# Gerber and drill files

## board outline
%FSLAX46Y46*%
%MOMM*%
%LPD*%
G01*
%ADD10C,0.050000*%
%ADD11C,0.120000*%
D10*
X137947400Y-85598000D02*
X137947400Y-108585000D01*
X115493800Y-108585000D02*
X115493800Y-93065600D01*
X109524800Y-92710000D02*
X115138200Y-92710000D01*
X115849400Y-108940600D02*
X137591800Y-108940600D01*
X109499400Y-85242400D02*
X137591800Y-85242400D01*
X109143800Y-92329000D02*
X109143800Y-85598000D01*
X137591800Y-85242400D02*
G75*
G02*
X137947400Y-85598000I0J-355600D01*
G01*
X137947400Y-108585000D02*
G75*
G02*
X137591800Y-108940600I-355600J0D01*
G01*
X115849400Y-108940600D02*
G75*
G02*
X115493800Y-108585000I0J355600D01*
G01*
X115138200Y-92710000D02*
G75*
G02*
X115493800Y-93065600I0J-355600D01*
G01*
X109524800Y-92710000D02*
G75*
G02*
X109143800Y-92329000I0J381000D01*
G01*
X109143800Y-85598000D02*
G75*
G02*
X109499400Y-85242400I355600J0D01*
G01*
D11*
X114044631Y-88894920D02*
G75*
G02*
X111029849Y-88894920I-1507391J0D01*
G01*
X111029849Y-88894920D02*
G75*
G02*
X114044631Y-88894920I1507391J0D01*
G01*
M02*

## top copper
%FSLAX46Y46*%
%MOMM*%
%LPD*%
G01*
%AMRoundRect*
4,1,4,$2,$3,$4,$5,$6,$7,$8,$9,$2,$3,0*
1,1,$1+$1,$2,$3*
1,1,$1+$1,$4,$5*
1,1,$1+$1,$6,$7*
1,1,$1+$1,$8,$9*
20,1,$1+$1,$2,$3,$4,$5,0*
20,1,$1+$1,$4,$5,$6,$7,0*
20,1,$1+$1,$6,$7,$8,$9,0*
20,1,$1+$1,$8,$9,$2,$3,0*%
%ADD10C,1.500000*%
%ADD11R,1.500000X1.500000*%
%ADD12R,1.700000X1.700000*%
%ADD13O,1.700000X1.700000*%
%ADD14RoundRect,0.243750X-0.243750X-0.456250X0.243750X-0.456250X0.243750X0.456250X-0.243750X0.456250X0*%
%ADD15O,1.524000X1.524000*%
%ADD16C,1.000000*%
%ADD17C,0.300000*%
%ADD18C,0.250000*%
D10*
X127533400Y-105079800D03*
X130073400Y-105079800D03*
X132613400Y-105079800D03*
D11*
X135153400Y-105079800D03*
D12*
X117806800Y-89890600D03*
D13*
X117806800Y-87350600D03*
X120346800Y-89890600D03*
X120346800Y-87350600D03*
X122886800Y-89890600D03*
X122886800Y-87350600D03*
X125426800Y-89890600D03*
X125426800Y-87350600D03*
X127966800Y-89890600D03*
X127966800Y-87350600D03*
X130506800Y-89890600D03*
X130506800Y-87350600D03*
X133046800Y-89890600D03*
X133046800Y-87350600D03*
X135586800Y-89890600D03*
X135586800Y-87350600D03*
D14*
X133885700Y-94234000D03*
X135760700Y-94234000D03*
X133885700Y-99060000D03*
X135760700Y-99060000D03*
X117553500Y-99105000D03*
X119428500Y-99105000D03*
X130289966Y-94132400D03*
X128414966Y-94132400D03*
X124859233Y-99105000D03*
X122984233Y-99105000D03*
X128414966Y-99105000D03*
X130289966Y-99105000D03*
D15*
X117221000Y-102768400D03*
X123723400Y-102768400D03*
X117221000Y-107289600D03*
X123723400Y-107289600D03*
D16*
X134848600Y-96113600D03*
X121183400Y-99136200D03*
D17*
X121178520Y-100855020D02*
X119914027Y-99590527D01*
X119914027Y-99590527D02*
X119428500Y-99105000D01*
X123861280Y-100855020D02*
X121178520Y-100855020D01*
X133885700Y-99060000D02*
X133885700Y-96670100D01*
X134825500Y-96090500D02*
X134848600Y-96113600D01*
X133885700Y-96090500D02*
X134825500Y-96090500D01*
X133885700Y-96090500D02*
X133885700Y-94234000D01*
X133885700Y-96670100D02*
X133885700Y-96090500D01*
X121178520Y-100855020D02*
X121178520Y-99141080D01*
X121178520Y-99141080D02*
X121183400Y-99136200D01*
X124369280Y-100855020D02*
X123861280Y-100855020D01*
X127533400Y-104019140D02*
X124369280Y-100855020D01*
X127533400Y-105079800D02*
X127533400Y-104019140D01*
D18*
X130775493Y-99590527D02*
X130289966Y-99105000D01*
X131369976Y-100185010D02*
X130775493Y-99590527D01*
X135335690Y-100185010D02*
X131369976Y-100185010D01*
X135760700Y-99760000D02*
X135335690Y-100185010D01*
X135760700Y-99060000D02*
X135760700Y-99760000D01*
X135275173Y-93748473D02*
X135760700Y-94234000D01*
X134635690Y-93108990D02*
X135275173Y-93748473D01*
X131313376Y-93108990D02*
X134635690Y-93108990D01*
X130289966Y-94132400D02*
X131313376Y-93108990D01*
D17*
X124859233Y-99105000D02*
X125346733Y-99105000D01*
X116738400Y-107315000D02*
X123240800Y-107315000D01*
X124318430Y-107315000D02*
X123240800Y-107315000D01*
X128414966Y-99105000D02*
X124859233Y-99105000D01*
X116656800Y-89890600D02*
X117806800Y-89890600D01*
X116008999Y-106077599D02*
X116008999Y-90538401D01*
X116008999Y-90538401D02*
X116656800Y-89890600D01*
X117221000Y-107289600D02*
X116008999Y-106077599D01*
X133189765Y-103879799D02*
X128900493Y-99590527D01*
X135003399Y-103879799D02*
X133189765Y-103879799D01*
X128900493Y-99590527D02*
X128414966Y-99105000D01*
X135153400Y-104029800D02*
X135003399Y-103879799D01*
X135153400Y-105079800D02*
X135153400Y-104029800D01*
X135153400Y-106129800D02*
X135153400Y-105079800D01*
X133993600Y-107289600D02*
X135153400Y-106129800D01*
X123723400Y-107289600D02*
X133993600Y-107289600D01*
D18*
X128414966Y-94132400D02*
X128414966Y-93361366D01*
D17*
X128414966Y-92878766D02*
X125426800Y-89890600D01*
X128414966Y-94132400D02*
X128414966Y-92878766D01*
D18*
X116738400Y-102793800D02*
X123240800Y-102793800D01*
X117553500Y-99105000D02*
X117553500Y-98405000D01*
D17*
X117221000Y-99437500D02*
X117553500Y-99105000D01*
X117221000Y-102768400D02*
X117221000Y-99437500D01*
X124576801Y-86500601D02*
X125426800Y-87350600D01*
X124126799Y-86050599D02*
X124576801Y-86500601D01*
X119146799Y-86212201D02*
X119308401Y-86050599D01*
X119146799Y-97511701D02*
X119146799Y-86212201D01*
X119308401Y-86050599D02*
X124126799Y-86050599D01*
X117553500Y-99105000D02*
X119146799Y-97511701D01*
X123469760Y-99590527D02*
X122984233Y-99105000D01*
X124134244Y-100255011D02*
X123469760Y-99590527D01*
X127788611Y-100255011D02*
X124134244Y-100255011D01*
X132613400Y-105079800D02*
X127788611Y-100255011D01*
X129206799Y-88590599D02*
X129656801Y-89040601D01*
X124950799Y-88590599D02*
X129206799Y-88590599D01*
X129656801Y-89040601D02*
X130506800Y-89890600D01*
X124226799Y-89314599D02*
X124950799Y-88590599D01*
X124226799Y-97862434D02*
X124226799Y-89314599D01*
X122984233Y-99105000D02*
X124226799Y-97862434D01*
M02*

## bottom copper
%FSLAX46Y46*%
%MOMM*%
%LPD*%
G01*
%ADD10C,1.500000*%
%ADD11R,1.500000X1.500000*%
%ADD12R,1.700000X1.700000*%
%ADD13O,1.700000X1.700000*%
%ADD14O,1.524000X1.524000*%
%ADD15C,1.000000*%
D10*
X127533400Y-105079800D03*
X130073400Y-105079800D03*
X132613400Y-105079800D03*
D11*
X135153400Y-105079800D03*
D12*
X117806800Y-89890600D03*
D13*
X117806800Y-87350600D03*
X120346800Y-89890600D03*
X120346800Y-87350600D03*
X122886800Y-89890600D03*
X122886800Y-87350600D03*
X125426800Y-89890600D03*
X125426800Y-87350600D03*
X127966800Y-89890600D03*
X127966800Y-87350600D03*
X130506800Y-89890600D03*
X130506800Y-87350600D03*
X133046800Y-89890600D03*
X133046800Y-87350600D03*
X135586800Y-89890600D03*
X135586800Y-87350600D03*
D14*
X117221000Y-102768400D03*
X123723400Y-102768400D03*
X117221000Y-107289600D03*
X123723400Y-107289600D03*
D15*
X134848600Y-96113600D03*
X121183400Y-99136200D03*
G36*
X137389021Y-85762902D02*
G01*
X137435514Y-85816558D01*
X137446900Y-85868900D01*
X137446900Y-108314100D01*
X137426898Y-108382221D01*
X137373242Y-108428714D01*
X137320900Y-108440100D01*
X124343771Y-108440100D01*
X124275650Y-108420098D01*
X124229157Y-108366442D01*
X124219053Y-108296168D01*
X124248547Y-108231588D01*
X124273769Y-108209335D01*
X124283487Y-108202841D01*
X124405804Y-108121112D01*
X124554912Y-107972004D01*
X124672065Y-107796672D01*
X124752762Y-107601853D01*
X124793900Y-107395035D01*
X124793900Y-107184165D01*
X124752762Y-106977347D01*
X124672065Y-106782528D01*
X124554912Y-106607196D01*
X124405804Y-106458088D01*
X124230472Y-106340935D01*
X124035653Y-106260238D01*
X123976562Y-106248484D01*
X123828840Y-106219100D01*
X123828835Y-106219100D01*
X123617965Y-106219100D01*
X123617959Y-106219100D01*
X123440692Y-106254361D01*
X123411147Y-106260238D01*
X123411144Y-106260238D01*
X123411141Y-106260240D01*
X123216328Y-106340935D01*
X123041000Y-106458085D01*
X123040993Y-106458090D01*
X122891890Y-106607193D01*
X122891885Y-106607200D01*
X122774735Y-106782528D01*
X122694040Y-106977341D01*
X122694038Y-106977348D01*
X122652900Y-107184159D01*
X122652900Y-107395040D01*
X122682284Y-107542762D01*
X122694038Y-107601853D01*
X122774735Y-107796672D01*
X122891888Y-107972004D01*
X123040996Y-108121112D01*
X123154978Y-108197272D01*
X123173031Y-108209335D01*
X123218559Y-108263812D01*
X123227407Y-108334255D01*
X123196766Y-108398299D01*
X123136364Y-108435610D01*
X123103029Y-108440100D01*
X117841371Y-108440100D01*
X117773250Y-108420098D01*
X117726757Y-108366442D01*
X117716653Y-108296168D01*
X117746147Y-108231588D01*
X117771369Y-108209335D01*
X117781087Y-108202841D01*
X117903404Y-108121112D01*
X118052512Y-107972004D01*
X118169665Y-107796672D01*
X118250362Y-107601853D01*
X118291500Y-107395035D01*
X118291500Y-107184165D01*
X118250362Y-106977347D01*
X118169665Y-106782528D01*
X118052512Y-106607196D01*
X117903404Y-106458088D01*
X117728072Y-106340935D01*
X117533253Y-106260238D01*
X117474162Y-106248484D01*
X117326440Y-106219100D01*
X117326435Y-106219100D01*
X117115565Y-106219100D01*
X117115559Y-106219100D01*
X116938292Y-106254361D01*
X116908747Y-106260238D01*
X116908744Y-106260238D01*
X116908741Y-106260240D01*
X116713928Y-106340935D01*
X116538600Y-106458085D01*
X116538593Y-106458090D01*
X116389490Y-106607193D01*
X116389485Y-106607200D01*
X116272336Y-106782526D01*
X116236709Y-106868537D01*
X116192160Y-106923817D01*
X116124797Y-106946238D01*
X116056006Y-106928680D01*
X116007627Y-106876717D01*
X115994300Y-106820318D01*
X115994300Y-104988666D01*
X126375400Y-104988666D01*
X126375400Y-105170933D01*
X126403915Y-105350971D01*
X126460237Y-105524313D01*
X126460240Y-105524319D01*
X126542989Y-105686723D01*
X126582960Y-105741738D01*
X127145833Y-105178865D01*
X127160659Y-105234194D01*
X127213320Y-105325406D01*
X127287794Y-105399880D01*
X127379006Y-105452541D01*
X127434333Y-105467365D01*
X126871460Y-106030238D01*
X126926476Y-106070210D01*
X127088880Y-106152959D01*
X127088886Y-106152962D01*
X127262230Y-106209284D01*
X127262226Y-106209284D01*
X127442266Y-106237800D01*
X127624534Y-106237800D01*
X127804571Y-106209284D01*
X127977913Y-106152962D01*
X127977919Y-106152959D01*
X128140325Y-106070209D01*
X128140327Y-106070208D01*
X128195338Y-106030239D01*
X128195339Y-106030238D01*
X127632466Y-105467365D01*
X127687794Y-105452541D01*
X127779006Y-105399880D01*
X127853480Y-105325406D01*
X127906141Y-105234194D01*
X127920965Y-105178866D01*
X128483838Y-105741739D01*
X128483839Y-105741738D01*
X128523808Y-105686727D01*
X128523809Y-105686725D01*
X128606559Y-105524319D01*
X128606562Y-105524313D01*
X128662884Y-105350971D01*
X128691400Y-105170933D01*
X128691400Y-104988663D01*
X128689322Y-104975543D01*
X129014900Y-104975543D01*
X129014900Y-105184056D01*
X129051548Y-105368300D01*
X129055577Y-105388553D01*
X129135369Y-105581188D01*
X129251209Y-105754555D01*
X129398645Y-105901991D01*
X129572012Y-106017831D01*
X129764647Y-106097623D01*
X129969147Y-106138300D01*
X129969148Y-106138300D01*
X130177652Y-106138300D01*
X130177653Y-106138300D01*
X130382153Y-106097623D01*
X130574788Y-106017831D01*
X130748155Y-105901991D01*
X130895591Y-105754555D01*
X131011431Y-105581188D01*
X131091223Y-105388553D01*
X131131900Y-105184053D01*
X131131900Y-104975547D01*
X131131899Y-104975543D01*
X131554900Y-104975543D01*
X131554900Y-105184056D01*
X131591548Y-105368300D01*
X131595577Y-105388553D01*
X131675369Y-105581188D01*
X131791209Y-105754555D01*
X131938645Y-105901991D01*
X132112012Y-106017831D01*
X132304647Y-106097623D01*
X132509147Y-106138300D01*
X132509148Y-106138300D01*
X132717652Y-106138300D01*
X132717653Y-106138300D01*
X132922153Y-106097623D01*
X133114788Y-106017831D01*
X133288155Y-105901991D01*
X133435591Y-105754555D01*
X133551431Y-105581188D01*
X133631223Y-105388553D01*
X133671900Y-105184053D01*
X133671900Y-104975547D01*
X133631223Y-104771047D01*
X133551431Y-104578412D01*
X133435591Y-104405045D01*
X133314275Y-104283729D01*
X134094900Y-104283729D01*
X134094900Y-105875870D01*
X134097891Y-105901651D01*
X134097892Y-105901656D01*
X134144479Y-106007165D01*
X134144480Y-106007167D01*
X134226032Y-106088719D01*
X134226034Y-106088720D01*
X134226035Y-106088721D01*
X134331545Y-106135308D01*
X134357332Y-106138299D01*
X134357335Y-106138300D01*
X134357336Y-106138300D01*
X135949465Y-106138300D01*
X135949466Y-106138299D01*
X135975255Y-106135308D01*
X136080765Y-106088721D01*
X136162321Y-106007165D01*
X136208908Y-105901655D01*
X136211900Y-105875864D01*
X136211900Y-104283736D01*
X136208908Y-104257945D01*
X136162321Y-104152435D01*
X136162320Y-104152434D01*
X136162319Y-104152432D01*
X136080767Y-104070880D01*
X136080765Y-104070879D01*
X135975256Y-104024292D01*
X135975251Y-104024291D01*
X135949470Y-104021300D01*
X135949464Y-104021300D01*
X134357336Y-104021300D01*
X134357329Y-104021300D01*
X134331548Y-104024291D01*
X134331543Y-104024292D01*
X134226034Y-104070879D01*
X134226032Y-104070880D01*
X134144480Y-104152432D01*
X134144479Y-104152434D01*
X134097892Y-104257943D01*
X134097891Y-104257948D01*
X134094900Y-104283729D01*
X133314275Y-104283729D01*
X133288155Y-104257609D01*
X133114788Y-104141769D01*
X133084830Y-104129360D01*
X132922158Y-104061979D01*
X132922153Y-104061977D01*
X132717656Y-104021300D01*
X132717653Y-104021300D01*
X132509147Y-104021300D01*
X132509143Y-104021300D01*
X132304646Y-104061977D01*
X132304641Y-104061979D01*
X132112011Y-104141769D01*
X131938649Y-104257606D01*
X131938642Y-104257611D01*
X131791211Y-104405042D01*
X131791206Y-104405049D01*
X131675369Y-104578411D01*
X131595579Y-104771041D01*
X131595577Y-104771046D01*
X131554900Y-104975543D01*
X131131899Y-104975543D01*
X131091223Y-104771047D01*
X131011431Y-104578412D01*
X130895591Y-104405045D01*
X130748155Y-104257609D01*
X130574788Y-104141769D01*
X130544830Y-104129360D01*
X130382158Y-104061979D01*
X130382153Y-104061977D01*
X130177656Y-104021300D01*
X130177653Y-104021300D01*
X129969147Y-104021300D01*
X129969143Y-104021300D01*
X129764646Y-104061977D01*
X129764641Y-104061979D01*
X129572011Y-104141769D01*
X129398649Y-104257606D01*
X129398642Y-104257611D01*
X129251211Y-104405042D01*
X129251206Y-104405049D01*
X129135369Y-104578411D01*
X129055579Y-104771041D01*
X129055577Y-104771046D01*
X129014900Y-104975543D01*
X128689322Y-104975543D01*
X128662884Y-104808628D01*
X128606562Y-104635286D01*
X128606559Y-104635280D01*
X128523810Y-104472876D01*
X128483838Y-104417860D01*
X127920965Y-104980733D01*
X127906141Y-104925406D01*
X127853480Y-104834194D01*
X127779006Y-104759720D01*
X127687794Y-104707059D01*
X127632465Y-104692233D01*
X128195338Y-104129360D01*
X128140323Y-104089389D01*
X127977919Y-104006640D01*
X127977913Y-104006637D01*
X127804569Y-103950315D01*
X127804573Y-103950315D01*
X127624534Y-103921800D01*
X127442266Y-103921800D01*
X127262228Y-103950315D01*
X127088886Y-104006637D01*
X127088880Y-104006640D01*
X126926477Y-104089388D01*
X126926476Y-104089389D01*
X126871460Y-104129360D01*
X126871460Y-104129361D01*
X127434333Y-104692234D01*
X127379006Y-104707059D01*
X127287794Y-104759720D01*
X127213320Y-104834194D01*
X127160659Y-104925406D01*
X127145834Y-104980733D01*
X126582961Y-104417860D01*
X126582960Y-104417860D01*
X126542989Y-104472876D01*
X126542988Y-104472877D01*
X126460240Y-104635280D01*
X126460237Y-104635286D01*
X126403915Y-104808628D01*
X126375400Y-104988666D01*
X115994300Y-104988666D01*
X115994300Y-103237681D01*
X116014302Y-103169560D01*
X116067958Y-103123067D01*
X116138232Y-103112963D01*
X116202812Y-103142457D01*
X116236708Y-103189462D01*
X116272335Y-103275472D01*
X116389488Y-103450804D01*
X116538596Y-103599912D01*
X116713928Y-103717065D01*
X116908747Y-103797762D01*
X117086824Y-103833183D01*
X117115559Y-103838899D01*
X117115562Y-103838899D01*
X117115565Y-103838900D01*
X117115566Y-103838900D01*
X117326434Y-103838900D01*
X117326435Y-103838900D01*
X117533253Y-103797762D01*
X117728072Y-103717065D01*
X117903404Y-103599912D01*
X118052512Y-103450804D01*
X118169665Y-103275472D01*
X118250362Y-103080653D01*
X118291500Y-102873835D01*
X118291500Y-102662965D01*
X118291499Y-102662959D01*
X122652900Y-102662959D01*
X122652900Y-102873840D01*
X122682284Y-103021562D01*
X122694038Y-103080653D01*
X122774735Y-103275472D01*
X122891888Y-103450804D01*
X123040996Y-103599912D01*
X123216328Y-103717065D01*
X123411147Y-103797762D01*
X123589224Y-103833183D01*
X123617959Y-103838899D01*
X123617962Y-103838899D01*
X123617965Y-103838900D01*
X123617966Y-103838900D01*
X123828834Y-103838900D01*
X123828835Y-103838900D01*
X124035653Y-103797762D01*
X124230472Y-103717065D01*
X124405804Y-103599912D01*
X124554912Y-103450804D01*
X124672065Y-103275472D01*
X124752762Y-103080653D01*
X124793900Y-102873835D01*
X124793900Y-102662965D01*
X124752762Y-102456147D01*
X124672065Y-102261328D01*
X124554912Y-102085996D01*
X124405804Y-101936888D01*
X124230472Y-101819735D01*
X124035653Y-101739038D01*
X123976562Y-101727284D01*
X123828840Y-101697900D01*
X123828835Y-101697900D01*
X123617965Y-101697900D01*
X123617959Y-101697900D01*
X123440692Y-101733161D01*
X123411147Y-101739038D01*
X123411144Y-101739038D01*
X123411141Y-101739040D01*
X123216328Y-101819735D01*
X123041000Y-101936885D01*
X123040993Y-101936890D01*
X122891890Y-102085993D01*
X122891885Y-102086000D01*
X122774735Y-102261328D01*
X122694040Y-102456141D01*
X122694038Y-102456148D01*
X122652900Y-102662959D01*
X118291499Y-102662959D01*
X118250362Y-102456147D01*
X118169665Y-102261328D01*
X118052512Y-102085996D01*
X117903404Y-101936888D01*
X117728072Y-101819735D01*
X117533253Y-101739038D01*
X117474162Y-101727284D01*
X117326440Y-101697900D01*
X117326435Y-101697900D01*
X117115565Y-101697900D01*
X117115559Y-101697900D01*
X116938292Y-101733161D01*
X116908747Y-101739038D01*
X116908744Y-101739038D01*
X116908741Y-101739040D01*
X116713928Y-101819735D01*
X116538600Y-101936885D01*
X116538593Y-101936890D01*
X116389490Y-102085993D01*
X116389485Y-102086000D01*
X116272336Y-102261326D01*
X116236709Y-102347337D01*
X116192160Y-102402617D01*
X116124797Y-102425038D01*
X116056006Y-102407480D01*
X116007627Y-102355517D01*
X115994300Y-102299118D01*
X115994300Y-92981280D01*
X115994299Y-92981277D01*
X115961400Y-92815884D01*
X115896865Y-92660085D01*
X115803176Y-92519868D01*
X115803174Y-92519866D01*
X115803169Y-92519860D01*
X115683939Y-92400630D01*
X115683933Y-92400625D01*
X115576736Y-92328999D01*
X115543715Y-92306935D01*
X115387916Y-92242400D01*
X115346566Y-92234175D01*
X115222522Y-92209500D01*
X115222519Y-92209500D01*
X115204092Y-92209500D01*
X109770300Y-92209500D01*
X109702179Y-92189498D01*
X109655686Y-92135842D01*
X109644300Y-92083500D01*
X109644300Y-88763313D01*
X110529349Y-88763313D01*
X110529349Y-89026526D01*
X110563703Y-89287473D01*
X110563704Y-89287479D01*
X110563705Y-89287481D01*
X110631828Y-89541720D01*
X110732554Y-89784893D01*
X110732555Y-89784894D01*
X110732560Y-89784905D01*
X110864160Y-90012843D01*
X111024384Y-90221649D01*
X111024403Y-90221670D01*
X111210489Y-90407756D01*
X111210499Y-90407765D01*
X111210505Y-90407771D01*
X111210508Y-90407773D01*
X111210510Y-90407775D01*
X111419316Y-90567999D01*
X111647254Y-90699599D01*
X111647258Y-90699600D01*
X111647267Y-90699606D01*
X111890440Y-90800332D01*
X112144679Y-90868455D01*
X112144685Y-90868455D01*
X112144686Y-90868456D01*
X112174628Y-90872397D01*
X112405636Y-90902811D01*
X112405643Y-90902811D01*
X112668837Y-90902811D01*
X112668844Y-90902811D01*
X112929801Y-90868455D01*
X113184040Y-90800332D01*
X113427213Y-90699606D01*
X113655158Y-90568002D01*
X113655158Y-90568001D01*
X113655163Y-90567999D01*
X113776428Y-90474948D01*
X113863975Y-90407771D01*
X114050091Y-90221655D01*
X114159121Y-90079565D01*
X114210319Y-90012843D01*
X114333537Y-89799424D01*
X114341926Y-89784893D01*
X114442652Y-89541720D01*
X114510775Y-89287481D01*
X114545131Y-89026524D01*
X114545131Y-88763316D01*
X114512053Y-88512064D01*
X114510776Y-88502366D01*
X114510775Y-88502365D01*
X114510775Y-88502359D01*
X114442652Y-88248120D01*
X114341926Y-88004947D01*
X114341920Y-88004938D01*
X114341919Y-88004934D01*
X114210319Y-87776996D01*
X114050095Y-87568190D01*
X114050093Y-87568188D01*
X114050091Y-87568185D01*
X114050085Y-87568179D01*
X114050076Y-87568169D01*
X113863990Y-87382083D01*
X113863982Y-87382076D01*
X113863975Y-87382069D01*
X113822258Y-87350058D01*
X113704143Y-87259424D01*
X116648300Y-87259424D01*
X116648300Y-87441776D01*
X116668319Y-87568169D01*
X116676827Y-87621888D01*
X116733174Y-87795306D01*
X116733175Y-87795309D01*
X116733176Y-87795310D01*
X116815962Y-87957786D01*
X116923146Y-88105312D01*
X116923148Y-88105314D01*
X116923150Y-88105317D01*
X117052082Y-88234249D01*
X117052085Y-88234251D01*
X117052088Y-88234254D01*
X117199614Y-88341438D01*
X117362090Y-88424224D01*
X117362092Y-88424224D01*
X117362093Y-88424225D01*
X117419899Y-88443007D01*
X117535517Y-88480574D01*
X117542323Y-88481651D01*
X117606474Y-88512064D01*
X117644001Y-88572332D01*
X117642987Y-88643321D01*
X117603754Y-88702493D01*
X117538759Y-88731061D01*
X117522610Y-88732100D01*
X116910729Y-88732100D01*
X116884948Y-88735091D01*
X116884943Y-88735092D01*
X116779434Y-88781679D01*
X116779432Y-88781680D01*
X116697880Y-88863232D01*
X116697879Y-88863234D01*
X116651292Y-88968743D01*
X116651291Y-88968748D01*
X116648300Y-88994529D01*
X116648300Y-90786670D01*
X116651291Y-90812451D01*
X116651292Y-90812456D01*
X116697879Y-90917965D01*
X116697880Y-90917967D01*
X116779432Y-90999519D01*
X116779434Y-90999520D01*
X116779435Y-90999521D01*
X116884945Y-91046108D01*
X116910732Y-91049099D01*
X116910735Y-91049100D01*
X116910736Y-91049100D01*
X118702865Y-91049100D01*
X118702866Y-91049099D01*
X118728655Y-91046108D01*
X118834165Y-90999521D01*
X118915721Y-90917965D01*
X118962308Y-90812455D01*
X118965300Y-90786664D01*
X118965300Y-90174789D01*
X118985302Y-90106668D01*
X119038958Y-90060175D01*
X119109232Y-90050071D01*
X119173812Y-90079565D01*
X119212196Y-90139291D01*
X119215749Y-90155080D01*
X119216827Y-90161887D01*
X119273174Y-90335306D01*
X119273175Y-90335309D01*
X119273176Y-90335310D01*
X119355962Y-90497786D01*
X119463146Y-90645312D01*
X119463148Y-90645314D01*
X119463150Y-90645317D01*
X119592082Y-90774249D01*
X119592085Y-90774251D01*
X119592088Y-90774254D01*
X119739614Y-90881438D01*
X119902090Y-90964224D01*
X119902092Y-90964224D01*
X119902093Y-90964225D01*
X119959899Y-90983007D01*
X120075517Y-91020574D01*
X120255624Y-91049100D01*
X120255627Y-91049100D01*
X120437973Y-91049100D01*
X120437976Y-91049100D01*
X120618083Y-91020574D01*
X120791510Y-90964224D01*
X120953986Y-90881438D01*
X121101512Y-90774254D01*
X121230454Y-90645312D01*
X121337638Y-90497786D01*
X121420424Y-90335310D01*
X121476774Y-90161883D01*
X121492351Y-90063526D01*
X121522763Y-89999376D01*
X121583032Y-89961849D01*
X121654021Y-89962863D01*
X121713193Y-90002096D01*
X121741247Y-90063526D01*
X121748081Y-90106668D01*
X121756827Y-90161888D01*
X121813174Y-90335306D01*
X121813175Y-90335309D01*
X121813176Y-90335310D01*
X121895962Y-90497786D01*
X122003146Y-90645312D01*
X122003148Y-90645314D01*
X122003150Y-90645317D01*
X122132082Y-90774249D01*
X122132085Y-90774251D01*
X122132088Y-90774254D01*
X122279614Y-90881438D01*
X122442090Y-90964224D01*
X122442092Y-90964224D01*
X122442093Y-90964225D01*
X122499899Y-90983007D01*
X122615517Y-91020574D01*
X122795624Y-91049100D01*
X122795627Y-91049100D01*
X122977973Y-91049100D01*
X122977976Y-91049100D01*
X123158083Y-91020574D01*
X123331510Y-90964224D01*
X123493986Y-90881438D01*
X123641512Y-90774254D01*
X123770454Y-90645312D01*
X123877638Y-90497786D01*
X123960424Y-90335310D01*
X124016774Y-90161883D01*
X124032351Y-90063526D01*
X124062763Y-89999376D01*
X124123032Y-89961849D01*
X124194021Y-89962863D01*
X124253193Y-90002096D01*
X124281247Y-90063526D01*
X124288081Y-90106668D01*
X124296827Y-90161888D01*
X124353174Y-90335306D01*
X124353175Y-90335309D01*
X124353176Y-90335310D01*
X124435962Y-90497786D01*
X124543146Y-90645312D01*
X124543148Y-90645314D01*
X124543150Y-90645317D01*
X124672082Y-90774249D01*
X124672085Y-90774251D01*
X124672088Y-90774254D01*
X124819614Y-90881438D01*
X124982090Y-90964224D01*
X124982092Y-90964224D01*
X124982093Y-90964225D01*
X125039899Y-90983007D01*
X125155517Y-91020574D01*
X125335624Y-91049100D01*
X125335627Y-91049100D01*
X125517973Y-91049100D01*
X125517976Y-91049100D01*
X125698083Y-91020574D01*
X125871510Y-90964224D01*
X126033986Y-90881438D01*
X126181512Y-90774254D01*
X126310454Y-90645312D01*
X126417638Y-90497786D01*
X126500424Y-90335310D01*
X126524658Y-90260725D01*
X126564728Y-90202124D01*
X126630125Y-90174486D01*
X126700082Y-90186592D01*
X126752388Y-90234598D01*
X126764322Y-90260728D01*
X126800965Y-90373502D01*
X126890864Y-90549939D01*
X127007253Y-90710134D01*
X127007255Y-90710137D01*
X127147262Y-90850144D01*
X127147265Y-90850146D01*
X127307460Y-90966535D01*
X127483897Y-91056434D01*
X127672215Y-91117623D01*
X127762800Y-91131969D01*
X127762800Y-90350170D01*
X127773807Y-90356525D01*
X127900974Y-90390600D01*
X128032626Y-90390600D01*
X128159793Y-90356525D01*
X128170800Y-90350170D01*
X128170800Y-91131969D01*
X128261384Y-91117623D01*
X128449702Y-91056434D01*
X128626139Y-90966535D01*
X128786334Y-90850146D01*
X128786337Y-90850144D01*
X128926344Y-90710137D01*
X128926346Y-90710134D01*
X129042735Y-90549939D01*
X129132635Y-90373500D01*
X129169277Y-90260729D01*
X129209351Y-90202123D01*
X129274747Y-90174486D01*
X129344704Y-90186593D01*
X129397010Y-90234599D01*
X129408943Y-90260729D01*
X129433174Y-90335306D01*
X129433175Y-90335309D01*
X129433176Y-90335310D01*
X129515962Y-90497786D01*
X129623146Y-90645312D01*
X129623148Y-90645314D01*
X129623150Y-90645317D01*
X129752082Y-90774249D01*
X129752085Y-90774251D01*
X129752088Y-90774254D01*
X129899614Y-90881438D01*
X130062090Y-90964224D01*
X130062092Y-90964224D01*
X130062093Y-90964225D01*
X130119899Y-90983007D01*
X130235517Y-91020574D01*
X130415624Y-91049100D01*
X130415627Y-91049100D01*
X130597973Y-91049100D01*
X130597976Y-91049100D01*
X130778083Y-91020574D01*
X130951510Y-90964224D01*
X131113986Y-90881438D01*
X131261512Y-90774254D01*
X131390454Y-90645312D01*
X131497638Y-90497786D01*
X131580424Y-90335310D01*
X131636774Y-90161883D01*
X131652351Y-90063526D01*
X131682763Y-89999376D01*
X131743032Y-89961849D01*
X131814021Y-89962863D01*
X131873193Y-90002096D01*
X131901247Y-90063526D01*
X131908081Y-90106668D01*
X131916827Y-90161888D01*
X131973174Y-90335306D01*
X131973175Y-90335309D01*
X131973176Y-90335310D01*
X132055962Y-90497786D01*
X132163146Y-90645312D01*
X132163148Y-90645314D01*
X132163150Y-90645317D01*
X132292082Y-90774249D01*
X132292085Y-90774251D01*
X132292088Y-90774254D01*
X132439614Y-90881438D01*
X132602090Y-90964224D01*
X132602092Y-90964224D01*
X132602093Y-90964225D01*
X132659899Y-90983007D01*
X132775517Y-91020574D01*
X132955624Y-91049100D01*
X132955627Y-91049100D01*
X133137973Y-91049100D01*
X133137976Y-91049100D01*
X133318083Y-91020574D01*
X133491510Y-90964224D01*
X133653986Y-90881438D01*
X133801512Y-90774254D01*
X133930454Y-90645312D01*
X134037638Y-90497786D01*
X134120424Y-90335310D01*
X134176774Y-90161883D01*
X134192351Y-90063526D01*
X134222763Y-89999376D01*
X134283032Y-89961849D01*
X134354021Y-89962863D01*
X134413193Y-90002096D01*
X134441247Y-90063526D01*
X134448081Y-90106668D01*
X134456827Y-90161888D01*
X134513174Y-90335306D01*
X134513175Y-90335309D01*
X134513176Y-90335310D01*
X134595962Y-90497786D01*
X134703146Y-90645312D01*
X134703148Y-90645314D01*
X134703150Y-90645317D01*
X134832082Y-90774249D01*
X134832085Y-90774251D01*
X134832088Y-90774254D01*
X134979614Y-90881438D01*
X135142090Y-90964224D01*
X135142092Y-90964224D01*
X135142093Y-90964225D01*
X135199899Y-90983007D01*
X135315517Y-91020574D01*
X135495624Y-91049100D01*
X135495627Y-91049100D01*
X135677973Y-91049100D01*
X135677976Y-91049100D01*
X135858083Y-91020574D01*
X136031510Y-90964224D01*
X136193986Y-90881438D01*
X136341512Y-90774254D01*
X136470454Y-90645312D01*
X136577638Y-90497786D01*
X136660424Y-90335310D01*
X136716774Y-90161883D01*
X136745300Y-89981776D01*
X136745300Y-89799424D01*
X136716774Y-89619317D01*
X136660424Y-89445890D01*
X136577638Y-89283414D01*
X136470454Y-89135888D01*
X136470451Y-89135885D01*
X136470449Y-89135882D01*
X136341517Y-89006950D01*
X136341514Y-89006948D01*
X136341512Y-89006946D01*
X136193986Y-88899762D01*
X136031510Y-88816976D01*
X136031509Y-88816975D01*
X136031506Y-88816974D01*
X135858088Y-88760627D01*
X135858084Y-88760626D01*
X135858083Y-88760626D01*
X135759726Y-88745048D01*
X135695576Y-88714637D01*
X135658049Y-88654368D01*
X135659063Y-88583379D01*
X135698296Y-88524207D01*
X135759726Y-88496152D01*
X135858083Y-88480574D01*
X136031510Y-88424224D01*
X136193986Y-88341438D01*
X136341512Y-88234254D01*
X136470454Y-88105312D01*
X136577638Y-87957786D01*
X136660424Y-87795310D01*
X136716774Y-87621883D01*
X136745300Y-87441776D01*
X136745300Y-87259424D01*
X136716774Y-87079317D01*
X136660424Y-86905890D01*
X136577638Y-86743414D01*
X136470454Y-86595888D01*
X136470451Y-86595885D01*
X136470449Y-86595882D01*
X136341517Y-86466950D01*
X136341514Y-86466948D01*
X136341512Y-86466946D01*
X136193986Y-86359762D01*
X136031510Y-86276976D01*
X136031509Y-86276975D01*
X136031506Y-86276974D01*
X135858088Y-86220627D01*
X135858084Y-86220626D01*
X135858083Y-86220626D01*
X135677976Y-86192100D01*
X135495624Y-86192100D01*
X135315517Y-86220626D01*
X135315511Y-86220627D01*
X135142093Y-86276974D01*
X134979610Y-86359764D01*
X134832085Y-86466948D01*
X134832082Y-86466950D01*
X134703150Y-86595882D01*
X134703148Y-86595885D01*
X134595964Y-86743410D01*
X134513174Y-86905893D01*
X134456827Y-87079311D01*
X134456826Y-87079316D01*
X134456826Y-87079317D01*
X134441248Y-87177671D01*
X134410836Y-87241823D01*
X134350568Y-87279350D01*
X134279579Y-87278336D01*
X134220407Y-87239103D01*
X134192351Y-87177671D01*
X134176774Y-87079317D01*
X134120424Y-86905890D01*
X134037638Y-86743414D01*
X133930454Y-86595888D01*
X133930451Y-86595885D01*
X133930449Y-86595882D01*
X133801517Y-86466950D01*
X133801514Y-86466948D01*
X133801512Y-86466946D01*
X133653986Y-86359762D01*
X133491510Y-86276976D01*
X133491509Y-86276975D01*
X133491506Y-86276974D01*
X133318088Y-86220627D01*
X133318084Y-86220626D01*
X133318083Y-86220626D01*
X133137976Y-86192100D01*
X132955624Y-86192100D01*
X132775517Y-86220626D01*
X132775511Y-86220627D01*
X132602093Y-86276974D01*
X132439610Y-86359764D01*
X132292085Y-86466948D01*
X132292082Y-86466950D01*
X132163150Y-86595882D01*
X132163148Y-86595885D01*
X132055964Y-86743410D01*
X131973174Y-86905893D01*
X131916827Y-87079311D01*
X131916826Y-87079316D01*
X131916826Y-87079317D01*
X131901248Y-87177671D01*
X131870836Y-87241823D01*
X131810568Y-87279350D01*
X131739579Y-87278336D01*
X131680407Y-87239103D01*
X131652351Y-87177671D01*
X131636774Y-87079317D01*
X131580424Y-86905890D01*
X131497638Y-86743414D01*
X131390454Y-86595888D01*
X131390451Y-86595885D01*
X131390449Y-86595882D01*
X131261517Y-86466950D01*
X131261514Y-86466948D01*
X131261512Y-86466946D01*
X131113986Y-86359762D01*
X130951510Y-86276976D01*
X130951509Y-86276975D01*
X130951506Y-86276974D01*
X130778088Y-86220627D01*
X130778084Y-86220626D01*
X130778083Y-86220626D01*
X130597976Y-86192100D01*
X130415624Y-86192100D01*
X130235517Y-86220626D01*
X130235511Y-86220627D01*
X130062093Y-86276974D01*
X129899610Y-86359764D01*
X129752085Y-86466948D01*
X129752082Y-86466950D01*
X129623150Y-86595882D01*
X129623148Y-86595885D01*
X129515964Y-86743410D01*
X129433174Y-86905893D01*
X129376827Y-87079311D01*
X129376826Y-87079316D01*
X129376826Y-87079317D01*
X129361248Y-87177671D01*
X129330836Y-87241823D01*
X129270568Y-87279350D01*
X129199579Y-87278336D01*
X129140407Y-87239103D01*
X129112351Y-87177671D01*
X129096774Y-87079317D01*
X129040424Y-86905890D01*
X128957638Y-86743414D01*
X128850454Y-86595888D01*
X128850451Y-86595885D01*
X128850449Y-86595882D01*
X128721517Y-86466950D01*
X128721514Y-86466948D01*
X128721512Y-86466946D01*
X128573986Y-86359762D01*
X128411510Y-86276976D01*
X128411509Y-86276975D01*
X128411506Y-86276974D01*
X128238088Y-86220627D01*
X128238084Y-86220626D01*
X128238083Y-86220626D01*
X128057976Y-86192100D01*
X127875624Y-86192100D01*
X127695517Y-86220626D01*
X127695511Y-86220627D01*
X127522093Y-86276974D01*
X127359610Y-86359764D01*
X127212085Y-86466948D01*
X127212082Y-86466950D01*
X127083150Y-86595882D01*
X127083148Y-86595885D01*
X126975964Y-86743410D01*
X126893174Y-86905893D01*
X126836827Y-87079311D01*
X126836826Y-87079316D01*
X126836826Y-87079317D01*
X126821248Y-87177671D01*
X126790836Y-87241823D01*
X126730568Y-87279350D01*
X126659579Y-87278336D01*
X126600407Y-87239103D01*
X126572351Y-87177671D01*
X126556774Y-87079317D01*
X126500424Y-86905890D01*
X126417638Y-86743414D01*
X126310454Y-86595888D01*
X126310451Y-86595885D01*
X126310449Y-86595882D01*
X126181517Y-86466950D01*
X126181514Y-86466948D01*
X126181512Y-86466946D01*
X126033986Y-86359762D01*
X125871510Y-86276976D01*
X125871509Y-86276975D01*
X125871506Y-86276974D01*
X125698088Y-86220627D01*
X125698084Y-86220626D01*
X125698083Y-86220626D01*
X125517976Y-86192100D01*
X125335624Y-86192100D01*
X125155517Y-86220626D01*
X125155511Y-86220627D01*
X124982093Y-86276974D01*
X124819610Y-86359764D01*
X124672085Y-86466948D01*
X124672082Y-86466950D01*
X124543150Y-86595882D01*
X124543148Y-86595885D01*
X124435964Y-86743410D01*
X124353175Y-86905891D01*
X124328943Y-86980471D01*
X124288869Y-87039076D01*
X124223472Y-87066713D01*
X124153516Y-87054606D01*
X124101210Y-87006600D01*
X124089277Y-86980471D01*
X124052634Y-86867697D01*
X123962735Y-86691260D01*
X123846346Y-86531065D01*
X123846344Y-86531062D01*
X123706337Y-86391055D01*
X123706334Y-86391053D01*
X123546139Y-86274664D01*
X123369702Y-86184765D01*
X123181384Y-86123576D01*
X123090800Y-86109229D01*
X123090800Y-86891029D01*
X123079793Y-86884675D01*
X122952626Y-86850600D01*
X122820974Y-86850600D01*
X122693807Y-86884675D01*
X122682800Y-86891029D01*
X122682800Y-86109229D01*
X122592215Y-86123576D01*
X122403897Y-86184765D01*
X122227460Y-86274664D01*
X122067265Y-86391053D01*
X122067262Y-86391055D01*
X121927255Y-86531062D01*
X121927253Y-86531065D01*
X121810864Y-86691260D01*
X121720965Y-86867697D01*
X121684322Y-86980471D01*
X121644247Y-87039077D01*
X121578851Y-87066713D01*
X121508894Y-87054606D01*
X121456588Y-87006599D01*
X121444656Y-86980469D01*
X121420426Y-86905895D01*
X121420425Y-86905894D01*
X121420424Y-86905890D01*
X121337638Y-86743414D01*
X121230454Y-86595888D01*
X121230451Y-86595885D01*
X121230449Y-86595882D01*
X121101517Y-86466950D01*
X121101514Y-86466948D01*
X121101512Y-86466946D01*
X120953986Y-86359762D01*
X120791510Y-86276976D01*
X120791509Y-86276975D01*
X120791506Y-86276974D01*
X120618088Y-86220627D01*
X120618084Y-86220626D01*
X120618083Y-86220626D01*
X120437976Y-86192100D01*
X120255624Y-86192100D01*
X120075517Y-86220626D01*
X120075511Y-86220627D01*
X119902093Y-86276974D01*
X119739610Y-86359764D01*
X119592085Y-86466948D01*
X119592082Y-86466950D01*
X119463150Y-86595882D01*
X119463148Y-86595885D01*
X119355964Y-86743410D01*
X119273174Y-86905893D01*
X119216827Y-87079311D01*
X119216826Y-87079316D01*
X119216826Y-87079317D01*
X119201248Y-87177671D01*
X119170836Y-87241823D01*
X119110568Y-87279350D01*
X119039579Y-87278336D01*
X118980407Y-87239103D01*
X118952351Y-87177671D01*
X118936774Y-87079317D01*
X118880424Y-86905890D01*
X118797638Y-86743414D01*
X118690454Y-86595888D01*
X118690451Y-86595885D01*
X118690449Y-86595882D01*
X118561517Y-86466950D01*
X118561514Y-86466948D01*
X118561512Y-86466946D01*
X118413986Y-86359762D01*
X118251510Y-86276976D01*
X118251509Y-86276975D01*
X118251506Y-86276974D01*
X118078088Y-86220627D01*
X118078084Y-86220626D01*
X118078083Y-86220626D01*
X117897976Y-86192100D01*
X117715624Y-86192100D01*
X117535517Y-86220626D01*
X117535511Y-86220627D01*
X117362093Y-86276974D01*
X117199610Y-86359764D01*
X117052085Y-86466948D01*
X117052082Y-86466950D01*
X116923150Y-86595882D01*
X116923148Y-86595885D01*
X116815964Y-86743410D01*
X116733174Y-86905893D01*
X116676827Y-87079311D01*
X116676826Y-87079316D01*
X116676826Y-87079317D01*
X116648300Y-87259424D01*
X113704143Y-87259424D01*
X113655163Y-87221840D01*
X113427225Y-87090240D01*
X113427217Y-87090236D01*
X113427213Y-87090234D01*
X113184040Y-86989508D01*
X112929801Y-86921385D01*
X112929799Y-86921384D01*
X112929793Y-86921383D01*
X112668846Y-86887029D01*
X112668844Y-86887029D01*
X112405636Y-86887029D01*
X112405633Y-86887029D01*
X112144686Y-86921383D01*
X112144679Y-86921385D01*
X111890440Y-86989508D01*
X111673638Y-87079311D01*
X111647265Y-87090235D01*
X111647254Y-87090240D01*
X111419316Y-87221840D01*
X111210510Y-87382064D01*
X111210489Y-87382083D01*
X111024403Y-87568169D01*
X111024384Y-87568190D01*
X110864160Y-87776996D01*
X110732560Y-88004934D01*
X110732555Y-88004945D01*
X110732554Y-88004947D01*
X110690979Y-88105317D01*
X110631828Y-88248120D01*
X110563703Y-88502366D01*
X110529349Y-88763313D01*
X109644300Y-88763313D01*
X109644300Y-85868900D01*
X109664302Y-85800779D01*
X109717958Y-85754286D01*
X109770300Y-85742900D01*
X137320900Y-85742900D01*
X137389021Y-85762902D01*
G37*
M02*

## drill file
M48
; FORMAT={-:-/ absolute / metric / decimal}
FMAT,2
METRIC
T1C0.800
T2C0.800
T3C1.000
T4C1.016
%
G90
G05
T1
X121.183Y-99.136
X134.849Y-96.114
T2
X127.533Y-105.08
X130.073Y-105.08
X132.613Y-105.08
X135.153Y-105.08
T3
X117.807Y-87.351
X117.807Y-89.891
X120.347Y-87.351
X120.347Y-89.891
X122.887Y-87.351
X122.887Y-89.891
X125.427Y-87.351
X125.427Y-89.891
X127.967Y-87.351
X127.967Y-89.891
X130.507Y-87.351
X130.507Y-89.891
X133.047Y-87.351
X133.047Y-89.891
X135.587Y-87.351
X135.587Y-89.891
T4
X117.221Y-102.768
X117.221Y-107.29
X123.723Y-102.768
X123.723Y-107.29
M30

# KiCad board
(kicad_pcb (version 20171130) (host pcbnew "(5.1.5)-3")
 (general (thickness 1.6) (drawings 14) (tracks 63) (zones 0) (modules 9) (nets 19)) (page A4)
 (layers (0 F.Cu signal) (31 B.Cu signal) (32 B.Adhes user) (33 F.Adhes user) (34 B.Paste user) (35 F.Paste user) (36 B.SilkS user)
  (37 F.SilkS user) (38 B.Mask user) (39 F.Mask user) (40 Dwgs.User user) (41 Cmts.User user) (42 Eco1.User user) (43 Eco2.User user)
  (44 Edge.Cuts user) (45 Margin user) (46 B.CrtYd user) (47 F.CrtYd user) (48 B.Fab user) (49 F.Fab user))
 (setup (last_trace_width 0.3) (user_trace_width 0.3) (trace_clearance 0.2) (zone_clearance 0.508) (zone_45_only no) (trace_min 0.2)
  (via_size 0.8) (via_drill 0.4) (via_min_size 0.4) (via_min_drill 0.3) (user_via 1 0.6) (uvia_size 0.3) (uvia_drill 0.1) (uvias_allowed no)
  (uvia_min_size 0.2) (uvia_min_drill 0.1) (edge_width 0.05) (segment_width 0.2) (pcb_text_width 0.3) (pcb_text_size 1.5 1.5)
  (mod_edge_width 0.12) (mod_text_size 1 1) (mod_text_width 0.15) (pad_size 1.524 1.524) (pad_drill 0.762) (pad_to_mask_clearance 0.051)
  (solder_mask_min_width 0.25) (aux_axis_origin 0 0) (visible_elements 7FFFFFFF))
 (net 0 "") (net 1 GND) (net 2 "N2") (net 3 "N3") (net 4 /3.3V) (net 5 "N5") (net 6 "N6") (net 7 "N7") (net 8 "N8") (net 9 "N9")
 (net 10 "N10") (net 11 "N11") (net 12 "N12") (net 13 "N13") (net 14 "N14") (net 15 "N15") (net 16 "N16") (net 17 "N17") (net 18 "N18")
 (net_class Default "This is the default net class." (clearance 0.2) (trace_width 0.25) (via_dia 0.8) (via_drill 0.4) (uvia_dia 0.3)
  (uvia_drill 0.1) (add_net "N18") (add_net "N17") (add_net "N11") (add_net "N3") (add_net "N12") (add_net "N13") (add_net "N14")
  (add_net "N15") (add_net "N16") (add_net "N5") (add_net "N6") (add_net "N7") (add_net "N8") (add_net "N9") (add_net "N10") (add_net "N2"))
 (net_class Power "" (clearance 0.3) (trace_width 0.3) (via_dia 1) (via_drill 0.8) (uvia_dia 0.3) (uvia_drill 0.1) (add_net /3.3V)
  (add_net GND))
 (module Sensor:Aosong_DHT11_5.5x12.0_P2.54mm (layer F.Cu) (at 135.1534 105.0798 270)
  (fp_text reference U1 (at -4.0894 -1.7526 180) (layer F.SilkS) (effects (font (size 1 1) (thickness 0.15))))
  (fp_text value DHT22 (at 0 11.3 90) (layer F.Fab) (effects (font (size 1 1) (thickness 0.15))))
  (pad 4 thru_hole circle (at 0 7.62 270) (size 1.5 1.5) (drill 0.8) (layers *.Cu *.Mask) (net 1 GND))
  (pad 3 thru_hole circle (at 0 5.08 270) (size 1.5 1.5) (drill 0.8) (layers *.Cu *.Mask) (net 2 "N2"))
  (pad 2 thru_hole circle (at 0 2.54 270) (size 1.5 1.5) (drill 0.8) (layers *.Cu *.Mask) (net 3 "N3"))
  (pad 1 thru_hole rect (at 0 0 270) (size 1.5 1.5) (drill 0.8) (layers *.Cu *.Mask) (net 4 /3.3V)))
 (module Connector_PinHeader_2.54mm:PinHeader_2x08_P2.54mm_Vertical (layer F.Cu) (at 117.8068 89.8906 90)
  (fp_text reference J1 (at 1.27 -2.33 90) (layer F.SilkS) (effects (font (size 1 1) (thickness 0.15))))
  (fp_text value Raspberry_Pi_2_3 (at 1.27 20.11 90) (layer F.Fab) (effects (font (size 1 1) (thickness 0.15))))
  (pad 1 thru_hole rect (at 0 0 90) (size 1.7 1.7) (drill 1) (layers *.Cu *.Mask) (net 4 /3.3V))
  (pad 2 thru_hole oval (at 2.54 0 90) (size 1.7 1.7) (drill 1) (layers *.Cu *.Mask) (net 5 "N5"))
  (pad 3 thru_hole oval (at 0 2.54 90) (size 1.7 1.7) (drill 1) (layers *.Cu *.Mask) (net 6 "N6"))
  (pad 4 thru_hole oval (at 2.54 2.54 90) (size 1.7 1.7) (drill 1) (layers *.Cu *.Mask) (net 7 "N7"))
  (pad 5 thru_hole oval (at 0 5.08 90) (size 1.7 1.7) (drill 1) (layers *.Cu *.Mask) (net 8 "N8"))
  (pad 6 thru_hole oval (at 2.54 5.08 90) (size 1.7 1.7) (drill 1) (layers *.Cu *.Mask) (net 1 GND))
  (pad 7 thru_hole oval (at 0 7.62 90) (size 1.7 1.7) (drill 1) (layers *.Cu *.Mask) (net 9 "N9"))
  (pad 8 thru_hole oval (at 2.54 7.62 90) (size 1.7 1.7) (drill 1) (layers *.Cu *.Mask) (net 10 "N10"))
  (pad 9 thru_hole oval (at 0 10.16 90) (size 1.7 1.7) (drill 1) (layers *.Cu *.Mask) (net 1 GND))
  (pad 10 thru_hole oval (at 2.54 10.16 90) (size 1.7 1.7) (drill 1) (layers *.Cu *.Mask) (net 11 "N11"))
  (pad 11 thru_hole oval (at 0 12.7 90) (size 1.7 1.7) (drill 1) (layers *.Cu *.Mask) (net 3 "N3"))
  (pad 12 thru_hole oval (at 2.54 12.7 90) (size 1.7 1.7) (drill 1) (layers *.Cu *.Mask) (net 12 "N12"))
  (pad 13 thru_hole oval (at 0 15.24 90) (size 1.7 1.7) (drill 1) (layers *.Cu *.Mask) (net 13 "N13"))
  (pad 14 thru_hole oval (at 2.54 15.24 90) (size 1.7 1.7) (drill 1) (layers *.Cu *.Mask) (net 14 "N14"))
  (pad 15 thru_hole oval (at 0 17.78 90) (size 1.7 1.7) (drill 1) (layers *.Cu *.Mask) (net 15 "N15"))
  (pad 16 thru_hole oval (at 2.54 17.78 90) (size 1.7 1.7) (drill 1) (layers *.Cu *.Mask) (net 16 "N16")))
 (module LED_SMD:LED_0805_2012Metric (layer F.Cu) (at 134.8232 94.234)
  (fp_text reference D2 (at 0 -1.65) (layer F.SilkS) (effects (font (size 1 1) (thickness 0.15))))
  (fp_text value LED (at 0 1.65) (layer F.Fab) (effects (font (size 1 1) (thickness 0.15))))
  (pad 1 smd roundrect (at -0.9375 0) (size 0.975 1.4) (layers F.Cu F.Paste F.Mask) (roundrect_rratio 0.25) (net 1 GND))
  (pad 2 smd roundrect (at 0.9375 0) (size 0.975 1.4) (layers F.Cu F.Paste F.Mask) (roundrect_rratio 0.25) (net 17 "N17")))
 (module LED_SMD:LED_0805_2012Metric (layer F.Cu) (at 134.8232 99.06)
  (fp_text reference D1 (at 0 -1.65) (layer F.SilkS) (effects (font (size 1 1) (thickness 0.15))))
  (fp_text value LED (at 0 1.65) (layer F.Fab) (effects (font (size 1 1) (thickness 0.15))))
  (pad 1 smd roundrect (at -0.9375 0) (size 0.975 1.4) (layers F.Cu F.Paste F.Mask) (roundrect_rratio 0.25) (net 1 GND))
  (pad 2 smd roundrect (at 0.9375 0) (size 0.975 1.4) (layers F.Cu F.Paste F.Mask) (roundrect_rratio 0.25) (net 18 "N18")))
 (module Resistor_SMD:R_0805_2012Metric (layer F.Cu) (at 118.491 99.105)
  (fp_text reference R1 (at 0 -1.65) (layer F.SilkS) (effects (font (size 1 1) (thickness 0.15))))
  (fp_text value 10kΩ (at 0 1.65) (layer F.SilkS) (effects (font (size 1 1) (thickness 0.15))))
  (pad 1 smd roundrect (at -0.9375 0) (size 0.975 1.4) (layers F.Cu F.Paste F.Mask) (roundrect_rratio 0.25) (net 10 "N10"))
  (pad 2 smd roundrect (at 0.9375 0) (size 0.975 1.4) (layers F.Cu F.Paste F.Mask) (roundrect_rratio 0.25) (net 1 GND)))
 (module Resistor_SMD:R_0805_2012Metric (layer F.Cu) (at 129.352466 94.1324)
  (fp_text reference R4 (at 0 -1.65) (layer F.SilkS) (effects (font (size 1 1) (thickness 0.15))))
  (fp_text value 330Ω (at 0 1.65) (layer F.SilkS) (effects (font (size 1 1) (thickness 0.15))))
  (pad 2 smd roundrect (at 0.9375 0) (size 0.975 1.4) (layers F.Cu F.Paste F.Mask) (roundrect_rratio 0.25) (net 17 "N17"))
  (pad 1 smd roundrect (at -0.9375 0) (size 0.975 1.4) (layers F.Cu F.Paste F.Mask) (roundrect_rratio 0.25) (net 9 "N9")))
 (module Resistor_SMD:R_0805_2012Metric (layer F.Cu) (at 123.921733 99.105)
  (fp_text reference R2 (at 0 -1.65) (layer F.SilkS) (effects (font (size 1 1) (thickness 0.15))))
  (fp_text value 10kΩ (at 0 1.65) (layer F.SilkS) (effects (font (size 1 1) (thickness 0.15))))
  (pad 2 smd roundrect (at 0.9375 0) (size 0.975 1.4) (layers F.Cu F.Paste F.Mask) (roundrect_rratio 0.25) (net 4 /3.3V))
  (pad 1 smd roundrect (at -0.9375 0) (size 0.975 1.4) (layers F.Cu F.Paste F.Mask) (roundrect_rratio 0.25) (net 3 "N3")))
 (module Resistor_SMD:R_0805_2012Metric (layer F.Cu) (at 129.352466 99.105)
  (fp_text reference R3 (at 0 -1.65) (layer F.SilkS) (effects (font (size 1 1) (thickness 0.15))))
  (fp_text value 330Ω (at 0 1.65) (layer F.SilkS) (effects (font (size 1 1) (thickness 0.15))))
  (pad 1 smd roundrect (at -0.9375 0) (size 0.975 1.4) (layers F.Cu F.Paste F.Mask) (roundrect_rratio 0.25) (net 4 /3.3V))
  (pad 2 smd roundrect (at 0.9375 0) (size 0.975 1.4) (layers F.Cu F.Paste F.Mask) (roundrect_rratio 0.25) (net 18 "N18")))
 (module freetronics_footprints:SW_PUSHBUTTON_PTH (layer F.Cu) (at 120.4722 105.029 180)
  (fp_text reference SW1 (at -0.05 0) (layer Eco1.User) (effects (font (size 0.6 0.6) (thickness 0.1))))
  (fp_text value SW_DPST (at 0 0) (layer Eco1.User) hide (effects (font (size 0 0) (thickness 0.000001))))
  (pad 2 thru_hole oval (at 3.2512 2.2606 180) (size 1.524 1.524) (drill 1.016) (layers *.Cu *.Mask) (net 10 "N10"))
  (pad 2 thru_hole oval (at -3.2512 2.2606 180) (size 1.524 1.524) (drill 1.016) (layers *.Cu *.Mask) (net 10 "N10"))
  (pad 1 thru_hole oval (at 3.2512 -2.2606 180) (size 1.524 1.524) (drill 1.016) (layers *.Cu *.Mask) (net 4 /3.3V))
  (pad 1 thru_hole oval (at -3.2512 -2.2606 180) (size 1.524 1.524) (drill 1.016) (layers *.Cu *.Mask) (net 4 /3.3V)))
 (gr_line (start 137.9474 85.598) (end 137.9474 108.585) (layer Edge.Cuts) (width 0.05))
 (gr_line (start 115.4938 108.585) (end 115.4938 93.0656) (layer Edge.Cuts) (width 0.05))
 (gr_line (start 109.5248 92.71) (end 115.1382 92.71) (layer Edge.Cuts) (width 0.05))
 (gr_line (start 115.8494 108.9406) (end 137.5918 108.9406) (layer Edge.Cuts) (width 0.05))
 (gr_line (start 109.4994 85.2424) (end 137.5918 85.2424) (layer Edge.Cuts) (width 0.05))
 (gr_line (start 109.1438 92.329) (end 109.1438 85.598) (layer Edge.Cuts) (width 0.05))
 (gr_arc (start 137.5918 85.598) (end 137.9474 85.598) (angle -90) (layer Edge.Cuts) (width 0.05))
 (gr_arc (start 137.5918 108.585) (end 137.5918 108.9406) (angle -90) (layer Edge.Cuts) (width 0.05))
 (gr_arc (start 115.8494 108.585) (end 115.4938 108.585) (angle -90) (layer Edge.Cuts) (width 0.05))
 (gr_arc (start 115.1382 93.0656) (end 115.4938 93.0656) (angle -90) (layer Edge.Cuts) (width 0.05))
 (gr_arc (start 109.5248 92.329) (end 109.1438 92.329) (angle -90) (layer Edge.Cuts) (width 0.05))
 (gr_arc (start 109.4994 85.598) (end 109.4994 85.2424) (angle -90) (layer Edge.Cuts) (width 0.05))
 (gr_circle (center 112.53724 88.89492) (end 114.044631 88.89492) (layer Edge.Cuts) (width 0.12))
 (segment (start 121.17852 100.85502) (end 119.914027 99.590527) (width 0.3) (layer F.Cu) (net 1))
 (segment (start 119.914027 99.590527) (end 119.4285 99.105) (width 0.3) (layer F.Cu) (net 1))
 (segment (start 123.86128 100.85502) (end 121.17852 100.85502) (width 0.3) (layer F.Cu) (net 1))
 (segment (start 133.8857 99.06) (end 133.8857 96.6701) (width 0.3) (layer F.Cu) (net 1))
 (via (at 134.8486 96.1136) (size 1) (drill 0.8) (layers F.Cu B.Cu) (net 1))
 (segment (start 134.8255 96.0905) (end 134.8486 96.1136) (width 0.3) (layer F.Cu) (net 1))
 (segment (start 133.8857 96.0905) (end 134.8255 96.0905) (width 0.3) (layer F.Cu) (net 1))
 (segment (start 133.8857 96.0905) (end 133.8857 94.234) (width 0.3) (layer F.Cu) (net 1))
 (segment (start 133.8857 96.6701) (end 133.8857 96.0905) (width 0.3) (layer F.Cu) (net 1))
 (via (at 121.1834 99.1362) (size 1) (drill 0.8) (layers F.Cu B.Cu) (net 1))
 (segment (start 121.17852 100.85502) (end 121.17852 99.14108) (width 0.3) (layer F.Cu) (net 1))
 (segment (start 121.17852 99.14108) (end 121.1834 99.1362) (width 0.3) (layer F.Cu) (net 1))
 (segment (start 124.36928 100.85502) (end 123.86128 100.85502) (width 0.3) (layer F.Cu) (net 1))
 (segment (start 127.5334 104.01914) (end 124.36928 100.85502) (width 0.3) (layer F.Cu) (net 1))
 (segment (start 127.5334 105.0798) (end 127.5334 104.01914) (width 0.3) (layer F.Cu) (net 1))
 (segment (start 130.775493 99.590527) (end 130.289966 99.105) (width 0.25) (layer F.Cu) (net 18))
 (segment (start 131.369976 100.18501) (end 130.775493 99.590527) (width 0.25) (layer F.Cu) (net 18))
 (segment (start 135.33569 100.18501) (end 131.369976 100.18501) (width 0.25) (layer F.Cu) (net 18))
 (segment (start 135.7607 99.76) (end 135.33569 100.18501) (width 0.25) (layer F.Cu) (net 18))
 (segment (start 135.7607 99.06) (end 135.7607 99.76) (width 0.25) (layer F.Cu) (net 18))
 (segment (start 135.275173 93.748473) (end 135.7607 94.234) (width 0.25) (layer F.Cu) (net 17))
 (segment (start 134.63569 93.10899) (end 135.275173 93.748473) (width 0.25) (layer F.Cu) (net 17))
 (segment (start 131.313376 93.10899) (end 134.63569 93.10899) (width 0.25) (layer F.Cu) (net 17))
 (segment (start 130.289966 94.1324) (end 131.313376 93.10899) (width 0.25) (layer F.Cu) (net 17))
 (segment (start 124.859233 99.105) (end 125.346733 99.105) (width 0.3) (layer F.Cu) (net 4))
 (segment (start 116.7384 107.315) (end 123.2408 107.315) (width 0.3) (layer F.Cu) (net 4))
 (segment (start 124.31843 107.315) (end 123.2408 107.315) (width 0.3) (layer F.Cu) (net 4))
 (segment (start 128.414966 99.105) (end 124.859233 99.105) (width 0.3) (layer F.Cu) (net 4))
 (segment (start 116.6568 89.8906) (end 117.8068 89.8906) (width 0.3) (layer F.Cu) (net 4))
 (segment (start 116.008999 106.077599) (end 116.008999 90.538401) (width 0.3) (layer F.Cu) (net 4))
 (segment (start 116.008999 90.538401) (end 116.6568 89.8906) (width 0.3) (layer F.Cu) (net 4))
 (segment (start 117.221 107.2896) (end 116.008999 106.077599) (width 0.3) (layer F.Cu) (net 4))
 (segment (start 133.189765 103.879799) (end 128.900493 99.590527) (width 0.3) (layer F.Cu) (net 4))
 (segment (start 135.003399 103.879799) (end 133.189765 103.879799) (width 0.3) (layer F.Cu) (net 4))
 (segment (start 128.900493 99.590527) (end 128.414966 99.105) (width 0.3) (layer F.Cu) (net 4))
 (segment (start 135.1534 104.0298) (end 135.003399 103.879799) (width 0.3) (layer F.Cu) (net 4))
 (segment (start 135.1534 105.0798) (end 135.1534 104.0298) (width 0.3) (layer F.Cu) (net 4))
 (segment (start 135.1534 106.1298) (end 135.1534 105.0798) (width 0.3) (layer F.Cu) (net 4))
 (segment (start 133.9936 107.2896) (end 135.1534 106.1298) (width 0.3) (layer F.Cu) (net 4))
 (segment (start 123.7234 107.2896) (end 133.9936 107.2896) (width 0.3) (layer F.Cu) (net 4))
 (segment (start 128.414966 94.1324) (end 128.414966 93.361366) (width 0.25) (layer F.Cu) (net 9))
 (segment (start 128.414966 92.878766) (end 125.4268 89.8906) (width 0.3) (layer F.Cu) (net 9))
 (segment (start 128.414966 94.1324) (end 128.414966 92.878766) (width 0.3) (layer F.Cu) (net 9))
 (segment (start 116.7384 102.7938) (end 123.2408 102.7938) (width 0.25) (layer F.Cu) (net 10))
 (segment (start 117.5535 99.105) (end 117.5535 98.405) (width 0.25) (layer F.Cu) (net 10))
 (segment (start 117.221 99.4375) (end 117.5535 99.105) (width 0.3) (layer F.Cu) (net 10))
 (segment (start 117.221 102.7684) (end 117.221 99.4375) (width 0.3) (layer F.Cu) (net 10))
 (segment (start 124.576801 86.500601) (end 125.4268 87.3506) (width 0.3) (layer F.Cu) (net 10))
 (segment (start 124.126799 86.050599) (end 124.576801 86.500601) (width 0.3) (layer F.Cu) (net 10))
 (segment (start 119.146799 86.212201) (end 119.308401 86.050599) (width 0.3) (layer F.Cu) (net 10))
 (segment (start 119.146799 97.511701) (end 119.146799 86.212201) (width 0.3) (layer F.Cu) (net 10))
 (segment (start 119.308401 86.050599) (end 124.126799 86.050599) (width 0.3) (layer F.Cu) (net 10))
 (segment (start 117.5535 99.105) (end 119.146799 97.511701) (width 0.3) (layer F.Cu) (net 10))
 (segment (start 123.46976 99.590527) (end 122.984233 99.105) (width 0.3) (layer F.Cu) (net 3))
 (segment (start 124.134244 100.255011) (end 123.46976 99.590527) (width 0.3) (layer F.Cu) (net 3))
 (segment (start 127.788611 100.255011) (end 124.134244 100.255011) (width 0.3) (layer F.Cu) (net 3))
 (segment (start 132.6134 105.0798) (end 127.788611 100.255011) (width 0.3) (layer F.Cu) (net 3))
 (segment (start 129.206799 88.590599) (end 129.656801 89.040601) (width 0.3) (layer F.Cu) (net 3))
 (segment (start 124.950799 88.590599) (end 129.206799 88.590599) (width 0.3) (layer F.Cu) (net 3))
 (segment (start 129.656801 89.040601) (end 130.5068 89.8906) (width 0.3) (layer F.Cu) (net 3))
 (segment (start 124.226799 89.314599) (end 124.950799 88.590599) (width 0.3) (layer F.Cu) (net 3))
 (segment (start 124.226799 97.862434) (end 124.226799 89.314599) (width 0.3) (layer F.Cu) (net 3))
 (segment (start 122.984233 99.105) (end 124.226799 97.862434) (width 0.3) (layer F.Cu) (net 3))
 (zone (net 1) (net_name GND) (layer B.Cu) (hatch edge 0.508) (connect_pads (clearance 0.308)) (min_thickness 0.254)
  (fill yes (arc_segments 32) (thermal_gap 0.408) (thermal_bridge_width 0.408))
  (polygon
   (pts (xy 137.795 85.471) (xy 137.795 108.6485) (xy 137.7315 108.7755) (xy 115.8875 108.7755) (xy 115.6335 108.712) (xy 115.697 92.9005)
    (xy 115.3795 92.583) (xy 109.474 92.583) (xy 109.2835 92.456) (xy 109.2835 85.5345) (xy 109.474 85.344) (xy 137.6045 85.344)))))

